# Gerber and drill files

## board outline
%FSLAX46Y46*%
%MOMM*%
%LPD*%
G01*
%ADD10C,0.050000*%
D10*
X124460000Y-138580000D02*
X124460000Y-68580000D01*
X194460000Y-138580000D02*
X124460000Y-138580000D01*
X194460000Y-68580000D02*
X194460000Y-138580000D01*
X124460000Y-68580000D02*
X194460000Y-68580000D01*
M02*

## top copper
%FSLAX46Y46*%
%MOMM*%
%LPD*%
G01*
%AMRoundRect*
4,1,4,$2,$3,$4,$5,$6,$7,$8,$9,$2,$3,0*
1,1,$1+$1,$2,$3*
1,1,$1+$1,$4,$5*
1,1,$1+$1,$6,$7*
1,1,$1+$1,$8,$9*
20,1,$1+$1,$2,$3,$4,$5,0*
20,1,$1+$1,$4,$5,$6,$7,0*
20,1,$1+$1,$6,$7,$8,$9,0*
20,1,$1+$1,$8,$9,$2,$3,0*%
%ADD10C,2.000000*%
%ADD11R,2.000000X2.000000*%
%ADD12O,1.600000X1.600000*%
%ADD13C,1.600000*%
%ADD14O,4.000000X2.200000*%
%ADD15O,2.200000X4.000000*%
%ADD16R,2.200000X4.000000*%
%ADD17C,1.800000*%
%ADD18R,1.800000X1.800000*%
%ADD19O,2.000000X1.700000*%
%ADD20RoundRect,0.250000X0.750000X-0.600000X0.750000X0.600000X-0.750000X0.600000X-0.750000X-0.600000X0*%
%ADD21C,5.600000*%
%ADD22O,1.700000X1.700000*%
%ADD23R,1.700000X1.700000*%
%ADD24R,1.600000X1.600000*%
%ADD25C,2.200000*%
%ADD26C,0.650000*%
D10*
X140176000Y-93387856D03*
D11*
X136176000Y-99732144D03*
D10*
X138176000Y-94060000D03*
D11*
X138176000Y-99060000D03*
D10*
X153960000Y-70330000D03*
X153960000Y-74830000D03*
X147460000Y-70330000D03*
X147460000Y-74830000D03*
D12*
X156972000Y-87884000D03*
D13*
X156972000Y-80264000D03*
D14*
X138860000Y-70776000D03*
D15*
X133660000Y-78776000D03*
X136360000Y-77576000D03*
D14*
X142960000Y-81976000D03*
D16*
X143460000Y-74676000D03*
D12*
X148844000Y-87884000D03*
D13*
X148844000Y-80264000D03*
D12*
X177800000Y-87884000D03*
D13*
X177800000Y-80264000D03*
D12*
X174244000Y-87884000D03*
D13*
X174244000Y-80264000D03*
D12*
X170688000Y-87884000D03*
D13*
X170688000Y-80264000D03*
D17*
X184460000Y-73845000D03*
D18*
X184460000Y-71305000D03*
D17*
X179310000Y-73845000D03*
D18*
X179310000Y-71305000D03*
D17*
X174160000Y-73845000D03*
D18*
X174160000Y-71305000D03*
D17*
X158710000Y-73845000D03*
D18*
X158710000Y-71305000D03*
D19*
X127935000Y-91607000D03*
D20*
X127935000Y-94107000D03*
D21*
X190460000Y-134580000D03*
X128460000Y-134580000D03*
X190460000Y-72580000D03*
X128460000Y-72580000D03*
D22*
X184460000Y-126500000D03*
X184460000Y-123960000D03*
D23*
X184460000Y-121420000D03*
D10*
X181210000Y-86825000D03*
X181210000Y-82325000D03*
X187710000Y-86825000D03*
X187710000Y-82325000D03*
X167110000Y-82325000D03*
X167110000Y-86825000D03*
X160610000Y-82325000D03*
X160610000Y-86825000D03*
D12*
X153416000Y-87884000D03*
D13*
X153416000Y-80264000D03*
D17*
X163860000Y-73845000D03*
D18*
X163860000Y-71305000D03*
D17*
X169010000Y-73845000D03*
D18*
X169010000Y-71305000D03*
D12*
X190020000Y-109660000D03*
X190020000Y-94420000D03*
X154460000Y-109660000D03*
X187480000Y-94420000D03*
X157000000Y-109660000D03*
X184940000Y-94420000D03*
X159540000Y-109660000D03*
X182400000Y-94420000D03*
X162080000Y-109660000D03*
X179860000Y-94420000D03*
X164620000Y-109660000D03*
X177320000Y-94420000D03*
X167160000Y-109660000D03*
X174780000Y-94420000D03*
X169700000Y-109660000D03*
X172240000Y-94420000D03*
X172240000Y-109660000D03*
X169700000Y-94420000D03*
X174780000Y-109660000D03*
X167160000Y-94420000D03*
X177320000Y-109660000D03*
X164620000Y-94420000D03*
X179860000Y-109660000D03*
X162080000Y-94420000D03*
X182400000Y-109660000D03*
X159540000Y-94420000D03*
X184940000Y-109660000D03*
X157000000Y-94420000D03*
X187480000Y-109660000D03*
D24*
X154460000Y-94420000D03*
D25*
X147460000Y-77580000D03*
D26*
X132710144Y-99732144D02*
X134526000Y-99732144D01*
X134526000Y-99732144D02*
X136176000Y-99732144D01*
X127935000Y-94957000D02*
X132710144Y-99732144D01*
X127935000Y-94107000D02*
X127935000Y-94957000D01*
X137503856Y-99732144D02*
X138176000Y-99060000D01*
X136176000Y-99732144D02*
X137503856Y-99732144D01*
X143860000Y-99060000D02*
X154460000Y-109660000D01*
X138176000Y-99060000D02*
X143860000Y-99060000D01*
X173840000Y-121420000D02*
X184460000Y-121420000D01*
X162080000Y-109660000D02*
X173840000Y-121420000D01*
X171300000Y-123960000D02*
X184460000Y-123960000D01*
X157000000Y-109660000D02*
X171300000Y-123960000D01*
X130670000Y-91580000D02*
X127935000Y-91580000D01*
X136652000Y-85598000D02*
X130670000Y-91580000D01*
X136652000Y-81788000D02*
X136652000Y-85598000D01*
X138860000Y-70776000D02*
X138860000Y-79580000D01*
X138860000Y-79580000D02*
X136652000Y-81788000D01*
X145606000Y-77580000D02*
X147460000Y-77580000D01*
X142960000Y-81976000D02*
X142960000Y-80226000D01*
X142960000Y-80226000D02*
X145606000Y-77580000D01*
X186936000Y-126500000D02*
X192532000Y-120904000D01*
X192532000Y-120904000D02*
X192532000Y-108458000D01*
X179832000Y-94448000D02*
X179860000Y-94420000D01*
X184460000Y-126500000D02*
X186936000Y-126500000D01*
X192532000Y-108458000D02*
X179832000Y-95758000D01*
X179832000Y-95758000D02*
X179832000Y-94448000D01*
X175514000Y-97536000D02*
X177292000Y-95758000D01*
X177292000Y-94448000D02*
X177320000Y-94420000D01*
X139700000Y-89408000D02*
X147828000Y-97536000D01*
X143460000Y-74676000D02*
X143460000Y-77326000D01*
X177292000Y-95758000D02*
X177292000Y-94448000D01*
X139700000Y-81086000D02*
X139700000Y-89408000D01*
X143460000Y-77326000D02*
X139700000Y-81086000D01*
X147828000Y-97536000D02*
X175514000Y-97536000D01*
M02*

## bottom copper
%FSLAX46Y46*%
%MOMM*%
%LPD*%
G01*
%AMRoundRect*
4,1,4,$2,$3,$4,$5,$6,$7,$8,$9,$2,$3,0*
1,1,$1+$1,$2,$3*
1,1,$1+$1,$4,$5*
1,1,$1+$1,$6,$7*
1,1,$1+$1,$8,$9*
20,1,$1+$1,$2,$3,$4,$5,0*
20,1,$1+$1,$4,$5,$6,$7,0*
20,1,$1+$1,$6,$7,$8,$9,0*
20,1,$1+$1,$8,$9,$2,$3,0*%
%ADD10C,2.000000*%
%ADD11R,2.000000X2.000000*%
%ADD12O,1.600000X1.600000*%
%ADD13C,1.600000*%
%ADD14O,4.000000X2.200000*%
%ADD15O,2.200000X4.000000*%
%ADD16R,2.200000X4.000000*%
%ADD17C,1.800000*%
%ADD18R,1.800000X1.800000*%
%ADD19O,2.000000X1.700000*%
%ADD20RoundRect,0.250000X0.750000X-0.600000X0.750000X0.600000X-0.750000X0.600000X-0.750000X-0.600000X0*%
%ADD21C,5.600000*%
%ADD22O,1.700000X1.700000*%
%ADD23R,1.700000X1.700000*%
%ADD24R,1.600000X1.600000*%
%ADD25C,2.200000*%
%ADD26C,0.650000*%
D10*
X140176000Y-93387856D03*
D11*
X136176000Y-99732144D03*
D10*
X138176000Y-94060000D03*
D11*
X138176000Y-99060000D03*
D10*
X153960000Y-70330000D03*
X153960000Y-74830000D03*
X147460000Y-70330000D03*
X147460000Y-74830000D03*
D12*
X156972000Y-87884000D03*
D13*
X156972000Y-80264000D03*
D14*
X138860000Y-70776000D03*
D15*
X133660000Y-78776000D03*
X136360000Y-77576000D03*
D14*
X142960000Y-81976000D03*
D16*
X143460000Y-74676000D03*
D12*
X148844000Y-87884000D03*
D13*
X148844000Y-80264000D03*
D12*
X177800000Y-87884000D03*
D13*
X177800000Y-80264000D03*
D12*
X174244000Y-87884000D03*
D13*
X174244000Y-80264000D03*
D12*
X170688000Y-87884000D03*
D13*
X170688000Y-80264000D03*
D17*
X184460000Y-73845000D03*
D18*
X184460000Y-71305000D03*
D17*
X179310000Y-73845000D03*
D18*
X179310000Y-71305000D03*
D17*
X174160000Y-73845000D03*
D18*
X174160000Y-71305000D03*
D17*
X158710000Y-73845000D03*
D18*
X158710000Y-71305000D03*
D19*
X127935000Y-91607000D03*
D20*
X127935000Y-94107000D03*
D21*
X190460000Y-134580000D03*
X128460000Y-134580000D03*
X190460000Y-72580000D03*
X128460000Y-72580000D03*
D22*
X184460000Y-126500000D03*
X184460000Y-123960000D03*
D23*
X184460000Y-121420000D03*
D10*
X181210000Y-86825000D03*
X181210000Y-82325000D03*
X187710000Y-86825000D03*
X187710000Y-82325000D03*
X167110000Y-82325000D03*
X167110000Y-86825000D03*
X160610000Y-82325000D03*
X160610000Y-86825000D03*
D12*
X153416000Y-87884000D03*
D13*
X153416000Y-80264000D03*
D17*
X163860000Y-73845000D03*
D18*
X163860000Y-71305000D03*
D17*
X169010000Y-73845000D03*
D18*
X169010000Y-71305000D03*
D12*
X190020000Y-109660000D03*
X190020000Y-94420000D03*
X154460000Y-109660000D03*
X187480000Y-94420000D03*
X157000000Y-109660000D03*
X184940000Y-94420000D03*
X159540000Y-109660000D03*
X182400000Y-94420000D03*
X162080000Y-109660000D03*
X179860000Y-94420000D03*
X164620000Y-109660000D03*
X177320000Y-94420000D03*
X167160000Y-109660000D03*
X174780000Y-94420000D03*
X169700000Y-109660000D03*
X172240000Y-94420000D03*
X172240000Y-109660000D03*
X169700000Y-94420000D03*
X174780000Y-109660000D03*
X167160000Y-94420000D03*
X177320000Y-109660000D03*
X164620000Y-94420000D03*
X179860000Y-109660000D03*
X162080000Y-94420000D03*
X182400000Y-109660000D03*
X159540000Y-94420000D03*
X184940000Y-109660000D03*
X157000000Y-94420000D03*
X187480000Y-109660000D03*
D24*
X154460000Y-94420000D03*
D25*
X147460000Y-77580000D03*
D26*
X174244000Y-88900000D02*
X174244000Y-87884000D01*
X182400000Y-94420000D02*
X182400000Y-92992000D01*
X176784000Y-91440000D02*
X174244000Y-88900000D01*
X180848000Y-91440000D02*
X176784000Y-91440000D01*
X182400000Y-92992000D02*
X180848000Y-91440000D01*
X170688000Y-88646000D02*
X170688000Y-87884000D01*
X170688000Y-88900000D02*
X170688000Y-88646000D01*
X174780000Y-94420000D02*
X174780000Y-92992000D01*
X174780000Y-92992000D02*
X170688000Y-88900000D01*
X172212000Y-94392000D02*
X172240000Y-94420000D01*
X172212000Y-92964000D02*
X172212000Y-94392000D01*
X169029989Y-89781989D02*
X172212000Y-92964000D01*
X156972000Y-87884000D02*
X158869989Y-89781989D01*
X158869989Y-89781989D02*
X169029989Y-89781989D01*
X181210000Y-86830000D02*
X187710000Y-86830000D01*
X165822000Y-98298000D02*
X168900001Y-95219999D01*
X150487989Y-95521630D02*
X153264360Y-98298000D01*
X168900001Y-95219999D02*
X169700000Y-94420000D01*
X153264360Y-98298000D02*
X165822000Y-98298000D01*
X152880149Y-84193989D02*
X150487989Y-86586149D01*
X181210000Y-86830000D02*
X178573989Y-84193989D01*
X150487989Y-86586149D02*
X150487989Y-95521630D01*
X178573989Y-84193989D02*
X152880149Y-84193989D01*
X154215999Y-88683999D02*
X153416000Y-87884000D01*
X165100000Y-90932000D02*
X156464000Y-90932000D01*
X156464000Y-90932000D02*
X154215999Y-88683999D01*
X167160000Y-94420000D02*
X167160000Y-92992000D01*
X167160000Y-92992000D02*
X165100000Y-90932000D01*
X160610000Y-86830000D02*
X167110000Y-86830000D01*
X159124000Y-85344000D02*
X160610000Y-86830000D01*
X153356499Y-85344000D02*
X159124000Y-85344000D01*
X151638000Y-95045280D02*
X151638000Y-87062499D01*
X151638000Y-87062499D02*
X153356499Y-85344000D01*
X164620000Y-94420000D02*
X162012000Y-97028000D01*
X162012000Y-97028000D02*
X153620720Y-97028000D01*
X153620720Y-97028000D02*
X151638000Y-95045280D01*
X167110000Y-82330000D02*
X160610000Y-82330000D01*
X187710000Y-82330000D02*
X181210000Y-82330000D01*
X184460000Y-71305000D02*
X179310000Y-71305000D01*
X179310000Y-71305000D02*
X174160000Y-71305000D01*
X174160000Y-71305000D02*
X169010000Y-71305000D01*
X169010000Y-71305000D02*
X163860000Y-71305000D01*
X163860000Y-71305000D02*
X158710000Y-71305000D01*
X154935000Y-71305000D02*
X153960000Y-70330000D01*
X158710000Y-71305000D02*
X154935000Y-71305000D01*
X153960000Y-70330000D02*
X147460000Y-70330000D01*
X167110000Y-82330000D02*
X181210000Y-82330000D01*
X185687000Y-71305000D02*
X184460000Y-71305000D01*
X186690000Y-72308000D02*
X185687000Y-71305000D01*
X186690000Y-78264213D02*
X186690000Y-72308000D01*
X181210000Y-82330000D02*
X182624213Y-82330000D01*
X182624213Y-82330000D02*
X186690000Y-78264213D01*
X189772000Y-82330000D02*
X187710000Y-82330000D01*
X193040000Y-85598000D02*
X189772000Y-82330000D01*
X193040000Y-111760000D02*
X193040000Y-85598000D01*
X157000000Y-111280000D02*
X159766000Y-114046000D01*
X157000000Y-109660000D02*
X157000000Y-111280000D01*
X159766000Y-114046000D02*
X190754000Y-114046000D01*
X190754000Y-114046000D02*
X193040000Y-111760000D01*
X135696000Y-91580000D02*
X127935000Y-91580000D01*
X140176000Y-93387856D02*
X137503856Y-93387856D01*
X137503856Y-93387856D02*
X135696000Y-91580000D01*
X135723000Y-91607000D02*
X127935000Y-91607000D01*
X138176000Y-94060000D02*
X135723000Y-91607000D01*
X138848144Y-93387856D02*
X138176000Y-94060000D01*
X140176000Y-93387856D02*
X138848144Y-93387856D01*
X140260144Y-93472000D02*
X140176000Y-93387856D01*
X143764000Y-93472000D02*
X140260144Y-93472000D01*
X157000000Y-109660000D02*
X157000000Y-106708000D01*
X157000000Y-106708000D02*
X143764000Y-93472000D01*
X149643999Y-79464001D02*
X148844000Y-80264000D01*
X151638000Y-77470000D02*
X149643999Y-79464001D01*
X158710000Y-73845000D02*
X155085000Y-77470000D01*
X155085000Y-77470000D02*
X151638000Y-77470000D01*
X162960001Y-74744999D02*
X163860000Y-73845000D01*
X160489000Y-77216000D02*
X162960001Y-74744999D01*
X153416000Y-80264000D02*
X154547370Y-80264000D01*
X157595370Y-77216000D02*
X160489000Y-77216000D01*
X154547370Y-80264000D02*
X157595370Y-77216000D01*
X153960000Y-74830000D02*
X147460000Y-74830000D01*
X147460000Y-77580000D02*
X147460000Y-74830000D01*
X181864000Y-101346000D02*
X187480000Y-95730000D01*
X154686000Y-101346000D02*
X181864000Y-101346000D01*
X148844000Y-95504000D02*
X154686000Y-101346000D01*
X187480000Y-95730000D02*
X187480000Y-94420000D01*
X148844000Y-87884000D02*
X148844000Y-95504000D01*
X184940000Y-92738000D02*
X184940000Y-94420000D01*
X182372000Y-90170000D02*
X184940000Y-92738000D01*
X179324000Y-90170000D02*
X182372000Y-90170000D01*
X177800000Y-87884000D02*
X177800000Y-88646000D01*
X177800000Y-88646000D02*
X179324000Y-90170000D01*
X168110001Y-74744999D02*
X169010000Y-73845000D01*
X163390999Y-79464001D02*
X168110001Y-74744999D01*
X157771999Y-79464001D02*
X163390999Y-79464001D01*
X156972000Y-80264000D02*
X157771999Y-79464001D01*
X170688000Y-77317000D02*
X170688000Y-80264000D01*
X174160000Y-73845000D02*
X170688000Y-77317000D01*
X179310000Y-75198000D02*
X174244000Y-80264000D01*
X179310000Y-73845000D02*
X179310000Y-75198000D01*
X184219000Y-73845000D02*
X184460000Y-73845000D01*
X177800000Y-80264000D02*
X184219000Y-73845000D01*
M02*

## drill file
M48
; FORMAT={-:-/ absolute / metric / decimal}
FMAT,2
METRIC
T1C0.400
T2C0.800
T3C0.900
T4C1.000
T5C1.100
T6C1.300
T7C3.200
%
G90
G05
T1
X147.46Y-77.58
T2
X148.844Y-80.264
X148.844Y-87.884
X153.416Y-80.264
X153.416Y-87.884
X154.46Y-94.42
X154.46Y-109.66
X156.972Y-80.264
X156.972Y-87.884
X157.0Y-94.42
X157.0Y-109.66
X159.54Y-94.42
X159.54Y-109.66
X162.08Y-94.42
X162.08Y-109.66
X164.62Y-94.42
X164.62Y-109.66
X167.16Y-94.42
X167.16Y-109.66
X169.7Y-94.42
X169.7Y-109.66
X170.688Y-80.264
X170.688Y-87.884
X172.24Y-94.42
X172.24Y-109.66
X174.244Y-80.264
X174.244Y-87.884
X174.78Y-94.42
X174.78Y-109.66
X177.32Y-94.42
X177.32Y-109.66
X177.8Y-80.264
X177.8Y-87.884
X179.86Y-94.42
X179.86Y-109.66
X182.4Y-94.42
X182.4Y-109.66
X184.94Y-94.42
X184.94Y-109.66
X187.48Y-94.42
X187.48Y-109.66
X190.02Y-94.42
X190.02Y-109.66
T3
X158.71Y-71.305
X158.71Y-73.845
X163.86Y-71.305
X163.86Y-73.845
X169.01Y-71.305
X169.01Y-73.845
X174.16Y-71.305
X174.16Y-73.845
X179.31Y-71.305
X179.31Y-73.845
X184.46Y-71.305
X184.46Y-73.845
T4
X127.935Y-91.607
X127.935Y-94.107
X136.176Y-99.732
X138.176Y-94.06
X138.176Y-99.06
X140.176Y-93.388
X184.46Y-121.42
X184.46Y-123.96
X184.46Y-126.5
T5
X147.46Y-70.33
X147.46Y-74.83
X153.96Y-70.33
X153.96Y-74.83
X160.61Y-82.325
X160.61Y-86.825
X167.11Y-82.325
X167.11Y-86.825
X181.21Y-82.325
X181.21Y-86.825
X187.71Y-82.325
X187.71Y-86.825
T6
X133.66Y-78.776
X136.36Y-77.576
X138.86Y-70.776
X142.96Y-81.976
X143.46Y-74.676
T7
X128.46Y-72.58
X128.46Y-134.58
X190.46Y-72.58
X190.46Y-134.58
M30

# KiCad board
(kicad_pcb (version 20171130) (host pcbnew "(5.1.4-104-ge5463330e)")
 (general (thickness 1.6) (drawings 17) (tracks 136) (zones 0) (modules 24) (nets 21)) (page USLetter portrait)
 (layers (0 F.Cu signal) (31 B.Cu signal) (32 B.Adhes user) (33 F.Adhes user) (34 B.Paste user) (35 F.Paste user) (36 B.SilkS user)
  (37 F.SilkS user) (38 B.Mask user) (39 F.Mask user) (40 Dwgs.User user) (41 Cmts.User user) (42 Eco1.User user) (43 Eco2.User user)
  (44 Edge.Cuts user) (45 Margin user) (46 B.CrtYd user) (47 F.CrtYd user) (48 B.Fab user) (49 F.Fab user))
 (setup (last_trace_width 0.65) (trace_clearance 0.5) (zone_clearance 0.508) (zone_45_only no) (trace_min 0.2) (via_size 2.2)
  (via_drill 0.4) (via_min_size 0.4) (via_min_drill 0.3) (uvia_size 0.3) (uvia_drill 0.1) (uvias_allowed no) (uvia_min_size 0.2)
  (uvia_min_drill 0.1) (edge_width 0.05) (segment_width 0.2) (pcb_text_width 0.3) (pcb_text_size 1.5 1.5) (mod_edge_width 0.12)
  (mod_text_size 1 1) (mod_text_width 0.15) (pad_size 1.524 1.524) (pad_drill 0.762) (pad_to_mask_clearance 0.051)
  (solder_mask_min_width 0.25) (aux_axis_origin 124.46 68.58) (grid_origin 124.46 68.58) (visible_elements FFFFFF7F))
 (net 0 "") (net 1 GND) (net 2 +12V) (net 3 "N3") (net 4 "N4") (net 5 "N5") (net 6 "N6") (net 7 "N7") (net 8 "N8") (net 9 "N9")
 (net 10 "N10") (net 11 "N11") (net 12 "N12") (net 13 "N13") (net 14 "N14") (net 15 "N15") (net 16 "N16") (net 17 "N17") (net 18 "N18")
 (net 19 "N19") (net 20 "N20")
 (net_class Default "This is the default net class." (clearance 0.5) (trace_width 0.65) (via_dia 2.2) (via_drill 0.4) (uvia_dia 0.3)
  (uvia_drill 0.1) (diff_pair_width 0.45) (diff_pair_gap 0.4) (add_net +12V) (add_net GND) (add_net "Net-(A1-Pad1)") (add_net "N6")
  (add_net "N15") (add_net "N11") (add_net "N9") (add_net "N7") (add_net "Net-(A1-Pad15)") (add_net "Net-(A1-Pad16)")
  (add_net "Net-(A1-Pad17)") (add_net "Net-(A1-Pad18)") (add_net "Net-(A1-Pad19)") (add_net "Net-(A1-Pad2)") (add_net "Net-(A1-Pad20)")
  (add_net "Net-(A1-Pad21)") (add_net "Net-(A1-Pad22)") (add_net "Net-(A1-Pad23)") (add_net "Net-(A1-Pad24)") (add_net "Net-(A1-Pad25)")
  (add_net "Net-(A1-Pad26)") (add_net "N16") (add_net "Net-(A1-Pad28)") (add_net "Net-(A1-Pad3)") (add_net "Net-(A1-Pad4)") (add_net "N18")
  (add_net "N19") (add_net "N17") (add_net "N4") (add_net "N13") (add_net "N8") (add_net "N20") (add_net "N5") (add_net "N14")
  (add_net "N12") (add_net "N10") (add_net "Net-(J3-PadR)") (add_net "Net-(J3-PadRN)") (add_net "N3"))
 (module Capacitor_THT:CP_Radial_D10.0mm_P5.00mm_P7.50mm (layer F.Cu) (at 138.176 99.06 90)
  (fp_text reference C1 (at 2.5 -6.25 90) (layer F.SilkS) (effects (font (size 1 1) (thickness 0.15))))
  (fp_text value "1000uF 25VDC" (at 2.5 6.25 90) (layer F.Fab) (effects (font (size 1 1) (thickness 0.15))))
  (pad 2 thru_hole circle (at 5.672144 2 90) (size 2 2) (drill 1) (layers *.Cu *.Mask) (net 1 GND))
  (pad 1 thru_hole rect (at -0.672144 -2 90) (size 2 2) (drill 1) (layers *.Cu *.Mask) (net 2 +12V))
  (pad 2 thru_hole circle (at 5 0 90) (size 2 2) (drill 1) (layers *.Cu *.Mask) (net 1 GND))
  (pad 1 thru_hole rect (at 0 0 90) (size 2 2) (drill 1) (layers *.Cu *.Mask) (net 2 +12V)))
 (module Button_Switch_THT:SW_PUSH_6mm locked (layer F.Cu) (at 147.46 70.33)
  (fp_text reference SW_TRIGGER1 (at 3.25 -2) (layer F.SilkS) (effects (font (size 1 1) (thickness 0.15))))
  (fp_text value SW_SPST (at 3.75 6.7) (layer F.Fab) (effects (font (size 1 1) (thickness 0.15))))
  (pad 1 thru_hole circle (at 6.5 0 90) (size 2 2) (drill 1.1) (layers *.Cu *.Mask) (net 1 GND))
  (pad 2 thru_hole circle (at 6.5 4.5 90) (size 2 2) (drill 1.1) (layers *.Cu *.Mask) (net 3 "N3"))
  (pad 1 thru_hole circle (at 0 0 90) (size 2 2) (drill 1.1) (layers *.Cu *.Mask) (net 1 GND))
  (pad 2 thru_hole circle (at 0 4.5 90) (size 2 2) (drill 1.1) (layers *.Cu *.Mask) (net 3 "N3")))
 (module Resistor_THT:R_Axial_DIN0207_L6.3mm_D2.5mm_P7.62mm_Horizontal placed (layer F.Cu) (at 156.972 80.264 270)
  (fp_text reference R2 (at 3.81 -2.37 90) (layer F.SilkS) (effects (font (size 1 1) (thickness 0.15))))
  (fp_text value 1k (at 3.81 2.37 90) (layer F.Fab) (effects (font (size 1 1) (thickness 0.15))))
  (pad 2 thru_hole oval (at 7.62 0 270) (size 1.6 1.6) (drill 0.8) (layers *.Cu *.Mask) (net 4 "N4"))
  (pad 1 thru_hole circle (at 0 0 270) (size 1.6 1.6) (drill 0.8) (layers *.Cu *.Mask) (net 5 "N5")))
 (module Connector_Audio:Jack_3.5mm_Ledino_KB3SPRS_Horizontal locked (layer B.Cu) (at 143.46 74.676 270)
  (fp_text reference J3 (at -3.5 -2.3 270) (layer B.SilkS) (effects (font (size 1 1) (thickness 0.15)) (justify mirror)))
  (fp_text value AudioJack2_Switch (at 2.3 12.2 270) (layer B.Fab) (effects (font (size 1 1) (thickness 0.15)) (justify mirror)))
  (pad S thru_hole oval (at -3.9 4.6 270) (size 2.2 4) (drill 1.3) (layers *.Cu *.Mask) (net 1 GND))
  (pad R thru_hole oval (at 4.1 9.8 270) (size 4 2.2) (drill 1.3) (layers *.Cu *.Mask))
  (pad RN thru_hole oval (at 2.9 7.1 270) (size 4 2.2) (drill 1.3) (layers *.Cu *.Mask))
  (pad TN thru_hole oval (at 7.3 0.5 180) (size 4 2.2) (drill 1.3) (layers *.Cu *.Mask) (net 3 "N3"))
  (pad T thru_hole rect (at 0 0 270) (size 4 2.2) (drill 1.3) (layers *.Cu *.Mask) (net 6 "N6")))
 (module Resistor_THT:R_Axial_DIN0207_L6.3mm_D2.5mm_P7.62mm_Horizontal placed (layer F.Cu) (at 148.844 80.264 270)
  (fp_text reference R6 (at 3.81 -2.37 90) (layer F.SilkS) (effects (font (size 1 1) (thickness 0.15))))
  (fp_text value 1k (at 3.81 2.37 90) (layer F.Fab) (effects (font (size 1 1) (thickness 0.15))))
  (pad 2 thru_hole oval (at 7.62 0 270) (size 1.6 1.6) (drill 0.8) (layers *.Cu *.Mask) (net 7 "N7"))
  (pad 1 thru_hole circle (at 0 0 270) (size 1.6 1.6) (drill 0.8) (layers *.Cu *.Mask) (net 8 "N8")))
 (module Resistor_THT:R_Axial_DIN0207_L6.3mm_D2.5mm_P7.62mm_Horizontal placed (layer F.Cu) (at 177.8 80.264 270)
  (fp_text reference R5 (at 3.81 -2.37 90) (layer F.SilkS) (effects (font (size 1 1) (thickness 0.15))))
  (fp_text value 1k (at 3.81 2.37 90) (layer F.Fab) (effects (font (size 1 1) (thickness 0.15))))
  (pad 2 thru_hole oval (at 7.62 0 270) (size 1.6 1.6) (drill 0.8) (layers *.Cu *.Mask) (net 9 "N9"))
  (pad 1 thru_hole circle (at 0 0 270) (size 1.6 1.6) (drill 0.8) (layers *.Cu *.Mask) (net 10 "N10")))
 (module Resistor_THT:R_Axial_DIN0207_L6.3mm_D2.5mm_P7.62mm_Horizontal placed (layer F.Cu) (at 174.244 80.264 270)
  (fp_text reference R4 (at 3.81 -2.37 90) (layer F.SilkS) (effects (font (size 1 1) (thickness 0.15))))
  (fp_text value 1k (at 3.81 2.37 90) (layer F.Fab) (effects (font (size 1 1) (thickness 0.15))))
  (pad 2 thru_hole oval (at 7.62 0 270) (size 1.6 1.6) (drill 0.8) (layers *.Cu *.Mask) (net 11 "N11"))
  (pad 1 thru_hole circle (at 0 0 270) (size 1.6 1.6) (drill 0.8) (layers *.Cu *.Mask) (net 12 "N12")))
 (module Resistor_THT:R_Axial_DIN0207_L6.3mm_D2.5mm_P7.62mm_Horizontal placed (layer F.Cu) (at 170.688 80.264 270)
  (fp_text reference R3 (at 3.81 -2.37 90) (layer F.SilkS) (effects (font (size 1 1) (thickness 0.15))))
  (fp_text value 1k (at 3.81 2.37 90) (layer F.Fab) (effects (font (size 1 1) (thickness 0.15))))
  (pad 2 thru_hole oval (at 7.62 0 270) (size 1.6 1.6) (drill 0.8) (layers *.Cu *.Mask) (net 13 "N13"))
  (pad 1 thru_hole circle (at 0 0 270) (size 1.6 1.6) (drill 0.8) (layers *.Cu *.Mask) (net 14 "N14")))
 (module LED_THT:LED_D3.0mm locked (layer F.Cu) (at 184.46 71.305 270)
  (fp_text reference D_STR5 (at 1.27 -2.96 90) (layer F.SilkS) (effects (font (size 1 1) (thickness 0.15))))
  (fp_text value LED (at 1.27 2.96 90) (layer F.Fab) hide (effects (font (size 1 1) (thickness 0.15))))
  (pad 2 thru_hole circle (at 2.54 0 270) (size 1.8 1.8) (drill 0.9) (layers *.Cu *.Mask) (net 10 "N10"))
  (pad 1 thru_hole rect (at 0 0 270) (size 1.8 1.8) (drill 0.9) (layers *.Cu *.Mask) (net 1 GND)))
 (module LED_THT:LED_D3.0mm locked (layer F.Cu) (at 179.31 71.305 270)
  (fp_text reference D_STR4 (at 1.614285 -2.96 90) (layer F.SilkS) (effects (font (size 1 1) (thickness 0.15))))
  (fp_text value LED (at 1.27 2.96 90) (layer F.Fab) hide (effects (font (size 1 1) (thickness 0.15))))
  (pad 2 thru_hole circle (at 2.54 0 270) (size 1.8 1.8) (drill 0.9) (layers *.Cu *.Mask) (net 12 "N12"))
  (pad 1 thru_hole rect (at 0 0 270) (size 1.8 1.8) (drill 0.9) (layers *.Cu *.Mask) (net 1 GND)))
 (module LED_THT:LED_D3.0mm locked (layer F.Cu) (at 174.16 71.305 270)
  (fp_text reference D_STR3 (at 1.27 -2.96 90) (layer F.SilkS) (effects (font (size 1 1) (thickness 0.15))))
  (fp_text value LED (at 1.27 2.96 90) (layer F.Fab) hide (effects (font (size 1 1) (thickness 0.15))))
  (pad 2 thru_hole circle (at 2.54 0 270) (size 1.8 1.8) (drill 0.9) (layers *.Cu *.Mask) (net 14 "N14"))
  (pad 1 thru_hole rect (at 0 0 270) (size 1.8 1.8) (drill 0.9) (layers *.Cu *.Mask) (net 1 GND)))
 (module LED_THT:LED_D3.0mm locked (layer F.Cu) (at 158.71 71.305 270)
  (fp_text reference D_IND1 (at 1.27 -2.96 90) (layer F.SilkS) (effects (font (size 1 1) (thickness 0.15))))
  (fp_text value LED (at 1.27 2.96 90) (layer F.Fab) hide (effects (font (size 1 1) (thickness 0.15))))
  (pad 2 thru_hole circle (at 2.54 0 270) (size 1.8 1.8) (drill 0.9) (layers *.Cu *.Mask) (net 8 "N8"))
  (pad 1 thru_hole rect (at 0 0 270) (size 1.8 1.8) (drill 0.9) (layers *.Cu *.Mask) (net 1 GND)))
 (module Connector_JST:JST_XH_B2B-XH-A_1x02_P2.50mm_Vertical (layer B.Cu) (at 127.935 94.107 90)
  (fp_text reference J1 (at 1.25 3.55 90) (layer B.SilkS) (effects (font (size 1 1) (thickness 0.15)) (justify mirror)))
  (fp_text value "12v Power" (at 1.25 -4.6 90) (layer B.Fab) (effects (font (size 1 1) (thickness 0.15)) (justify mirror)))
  (pad 2 thru_hole oval (at 2.5 0 90) (size 1.7 2) (drill 1) (layers *.Cu *.Mask) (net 1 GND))
  (pad 1 thru_hole roundrect (at 0 0 90) (size 1.7 2) (drill 1) (layers *.Cu *.Mask) (roundrect_rratio 0.147059) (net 2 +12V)))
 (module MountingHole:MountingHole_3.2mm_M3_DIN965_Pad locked (layer F.Cu) (at 190.46 134.58)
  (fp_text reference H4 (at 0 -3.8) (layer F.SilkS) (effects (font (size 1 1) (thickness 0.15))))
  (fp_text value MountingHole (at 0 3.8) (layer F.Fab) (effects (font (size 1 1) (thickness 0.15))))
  (pad 1 thru_hole circle (at 0 0) (size 5.6 5.6) (drill 3.2) (layers *.Cu *.Mask)))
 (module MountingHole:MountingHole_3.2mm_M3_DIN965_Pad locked (layer F.Cu) (at 128.46 134.58)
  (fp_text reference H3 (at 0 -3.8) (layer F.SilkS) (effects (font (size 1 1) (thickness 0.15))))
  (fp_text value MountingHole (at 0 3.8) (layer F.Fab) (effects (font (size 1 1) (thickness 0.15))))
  (pad 1 thru_hole circle (at 0 0) (size 5.6 5.6) (drill 3.2) (layers *.Cu *.Mask)))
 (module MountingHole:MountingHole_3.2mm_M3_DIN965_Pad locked (layer F.Cu) (at 190.46 72.58)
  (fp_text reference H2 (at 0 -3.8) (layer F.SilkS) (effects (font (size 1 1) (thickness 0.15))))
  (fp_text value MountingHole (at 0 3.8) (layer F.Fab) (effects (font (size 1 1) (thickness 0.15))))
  (pad 1 thru_hole circle (at 0 0) (size 5.6 5.6) (drill 3.2) (layers *.Cu *.Mask)))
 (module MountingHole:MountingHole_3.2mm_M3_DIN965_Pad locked (layer F.Cu) (at 128.46 72.58)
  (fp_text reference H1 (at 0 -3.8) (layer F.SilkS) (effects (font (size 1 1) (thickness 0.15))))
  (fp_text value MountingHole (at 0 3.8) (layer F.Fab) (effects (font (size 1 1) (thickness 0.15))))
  (pad 1 thru_hole circle (at 0 0) (size 5.6 5.6) (drill 3.2) (layers *.Cu *.Mask)))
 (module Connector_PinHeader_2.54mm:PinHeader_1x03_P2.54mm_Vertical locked (layer B.Cu) (at 184.46 121.42 180)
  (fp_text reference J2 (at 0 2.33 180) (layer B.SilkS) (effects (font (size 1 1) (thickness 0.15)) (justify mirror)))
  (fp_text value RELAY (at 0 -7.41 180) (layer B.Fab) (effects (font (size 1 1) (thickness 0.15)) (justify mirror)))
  (pad 3 thru_hole oval (at 0 -5.08 180) (size 1.7 1.7) (drill 1) (layers *.Cu *.Mask) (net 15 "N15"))
  (pad 2 thru_hole oval (at 0 -2.54 180) (size 1.7 1.7) (drill 1) (layers *.Cu *.Mask) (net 1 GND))
  (pad 1 thru_hole rect (at 0 0 180) (size 1.7 1.7) (drill 1) (layers *.Cu *.Mask) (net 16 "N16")))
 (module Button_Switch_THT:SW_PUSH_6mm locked (layer F.Cu) (at 187.71 86.825 180)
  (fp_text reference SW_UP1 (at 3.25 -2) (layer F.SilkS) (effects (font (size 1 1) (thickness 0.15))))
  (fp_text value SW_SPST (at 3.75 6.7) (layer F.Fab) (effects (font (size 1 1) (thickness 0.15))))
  (pad 1 thru_hole circle (at 6.5 0 270) (size 2 2) (drill 1.1) (layers *.Cu *.Mask) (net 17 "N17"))
  (pad 2 thru_hole circle (at 6.5 4.5 270) (size 2 2) (drill 1.1) (layers *.Cu *.Mask) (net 1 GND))
  (pad 1 thru_hole circle (at 0 0 270) (size 2 2) (drill 1.1) (layers *.Cu *.Mask) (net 17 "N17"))
  (pad 2 thru_hole circle (at 0 4.5 270) (size 2 2) (drill 1.1) (layers *.Cu *.Mask) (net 1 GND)))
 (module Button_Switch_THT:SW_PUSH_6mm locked (layer F.Cu) (at 167.11 86.825 180)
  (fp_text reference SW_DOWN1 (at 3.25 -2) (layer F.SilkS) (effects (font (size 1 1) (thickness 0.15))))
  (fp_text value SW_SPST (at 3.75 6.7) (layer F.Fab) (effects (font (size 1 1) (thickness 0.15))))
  (pad 2 thru_hole circle (at 0 4.5 270) (size 2 2) (drill 1.1) (layers *.Cu *.Mask) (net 1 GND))
  (pad 1 thru_hole circle (at 0 0 270) (size 2 2) (drill 1.1) (layers *.Cu *.Mask) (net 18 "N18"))
  (pad 2 thru_hole circle (at 6.5 4.5 270) (size 2 2) (drill 1.1) (layers *.Cu *.Mask) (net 1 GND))
  (pad 1 thru_hole circle (at 6.5 0 270) (size 2 2) (drill 1.1) (layers *.Cu *.Mask) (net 18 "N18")))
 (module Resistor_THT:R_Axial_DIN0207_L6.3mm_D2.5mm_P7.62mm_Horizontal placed (layer F.Cu) (at 153.416 80.264 270)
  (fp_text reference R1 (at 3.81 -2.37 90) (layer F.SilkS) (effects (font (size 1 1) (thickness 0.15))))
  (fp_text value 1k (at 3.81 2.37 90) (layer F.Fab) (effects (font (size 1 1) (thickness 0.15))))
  (pad 2 thru_hole oval (at 7.62 0 270) (size 1.6 1.6) (drill 0.8) (layers *.Cu *.Mask) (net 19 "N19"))
  (pad 1 thru_hole circle (at 0 0 270) (size 1.6 1.6) (drill 0.8) (layers *.Cu *.Mask) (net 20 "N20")))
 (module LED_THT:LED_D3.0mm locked (layer F.Cu) (at 163.86 71.305 270)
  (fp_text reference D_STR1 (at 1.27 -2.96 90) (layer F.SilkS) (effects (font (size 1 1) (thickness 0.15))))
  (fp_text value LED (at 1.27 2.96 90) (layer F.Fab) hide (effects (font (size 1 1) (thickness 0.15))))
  (pad 2 thru_hole circle (at 2.54 0 270) (size 1.8 1.8) (drill 0.9) (layers *.Cu *.Mask) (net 20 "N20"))
  (pad 1 thru_hole rect (at 0 0 270) (size 1.8 1.8) (drill 0.9) (layers *.Cu *.Mask) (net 1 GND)))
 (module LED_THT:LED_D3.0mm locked (layer F.Cu) (at 169.01 71.305 270)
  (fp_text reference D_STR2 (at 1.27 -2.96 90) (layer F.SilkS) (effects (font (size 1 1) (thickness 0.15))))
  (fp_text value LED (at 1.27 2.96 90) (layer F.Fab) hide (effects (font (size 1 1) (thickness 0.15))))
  (pad 2 thru_hole circle (at 2.54 0 270) (size 1.8 1.8) (drill 0.9) (layers *.Cu *.Mask) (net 5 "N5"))
  (pad 1 thru_hole rect (at 0 0 270) (size 1.8 1.8) (drill 0.9) (layers *.Cu *.Mask) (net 1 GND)))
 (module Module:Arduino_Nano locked (layer B.Cu) (at 154.46 94.42 270)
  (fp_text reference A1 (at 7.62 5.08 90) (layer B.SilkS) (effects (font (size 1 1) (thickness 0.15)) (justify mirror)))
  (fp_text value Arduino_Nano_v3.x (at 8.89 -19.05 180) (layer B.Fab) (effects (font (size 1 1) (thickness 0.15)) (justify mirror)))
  (pad 16 thru_hole oval (at 15.24 -35.56 270) (size 1.6 1.6) (drill 0.8) (layers *.Cu *.Mask))
  (pad 15 thru_hole oval (at 0 -35.56 270) (size 1.6 1.6) (drill 0.8) (layers *.Cu *.Mask))
  (pad 30 thru_hole oval (at 15.24 0 270) (size 1.6 1.6) (drill 0.8) (layers *.Cu *.Mask) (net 2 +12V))
  (pad 14 thru_hole oval (at 0 -33.02 270) (size 1.6 1.6) (drill 0.8) (layers *.Cu *.Mask) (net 7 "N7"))
  (pad 29 thru_hole oval (at 15.24 -2.54 270) (size 1.6 1.6) (drill 0.8) (layers *.Cu *.Mask) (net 1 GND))
  (pad 13 thru_hole oval (at 0 -30.48 270) (size 1.6 1.6) (drill 0.8) (layers *.Cu *.Mask) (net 9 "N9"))
  (pad 28 thru_hole oval (at 15.24 -5.08 270) (size 1.6 1.6) (drill 0.8) (layers *.Cu *.Mask))
  (pad 12 thru_hole oval (at 0 -27.94 270) (size 1.6 1.6) (drill 0.8) (layers *.Cu *.Mask) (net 11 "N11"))
  (pad 27 thru_hole oval (at 15.24 -7.62 270) (size 1.6 1.6) (drill 0.8) (layers *.Cu *.Mask) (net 16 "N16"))
  (pad 11 thru_hole oval (at 0 -25.4 270) (size 1.6 1.6) (drill 0.8) (layers *.Cu *.Mask) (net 15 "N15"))
  (pad 26 thru_hole oval (at 15.24 -10.16 270) (size 1.6 1.6) (drill 0.8) (layers *.Cu *.Mask))
  (pad 10 thru_hole oval (at 0 -22.86 270) (size 1.6 1.6) (drill 0.8) (layers *.Cu *.Mask) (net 6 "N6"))
  (pad 25 thru_hole oval (at 15.24 -12.7 270) (size 1.6 1.6) (drill 0.8) (layers *.Cu *.Mask))
  (pad 9 thru_hole oval (at 0 -20.32 270) (size 1.6 1.6) (drill 0.8) (layers *.Cu *.Mask) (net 13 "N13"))
  (pad 24 thru_hole oval (at 15.24 -15.24 270) (size 1.6 1.6) (drill 0.8) (layers *.Cu *.Mask))
  (pad 8 thru_hole oval (at 0 -17.78 270) (size 1.6 1.6) (drill 0.8) (layers *.Cu *.Mask) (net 4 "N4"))
  (pad 23 thru_hole oval (at 15.24 -17.78 270) (size 1.6 1.6) (drill 0.8) (layers *.Cu *.Mask))
  (pad 7 thru_hole oval (at 0 -15.24 270) (size 1.6 1.6) (drill 0.8) (layers *.Cu *.Mask) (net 17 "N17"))
  (pad 22 thru_hole oval (at 15.24 -20.32 270) (size 1.6 1.6) (drill 0.8) (layers *.Cu *.Mask))
  (pad 6 thru_hole oval (at 0 -12.7 270) (size 1.6 1.6) (drill 0.8) (layers *.Cu *.Mask) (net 19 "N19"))
  (pad 21 thru_hole oval (at 15.24 -22.86 270) (size 1.6 1.6) (drill 0.8) (layers *.Cu *.Mask))
  (pad 5 thru_hole oval (at 0 -10.16 270) (size 1.6 1.6) (drill 0.8) (layers *.Cu *.Mask) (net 18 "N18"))
  (pad 20 thru_hole oval (at 15.24 -25.4 270) (size 1.6 1.6) (drill 0.8) (layers *.Cu *.Mask))
  (pad 4 thru_hole oval (at 0 -7.62 270) (size 1.6 1.6) (drill 0.8) (layers *.Cu *.Mask))
  (pad 19 thru_hole oval (at 15.24 -27.94 270) (size 1.6 1.6) (drill 0.8) (layers *.Cu *.Mask))
  (pad 3 thru_hole oval (at 0 -5.08 270) (size 1.6 1.6) (drill 0.8) (layers *.Cu *.Mask))
  (pad 18 thru_hole oval (at 15.24 -30.48 270) (size 1.6 1.6) (drill 0.8) (layers *.Cu *.Mask))
  (pad 2 thru_hole oval (at 0 -2.54 270) (size 1.6 1.6) (drill 0.8) (layers *.Cu *.Mask))
  (pad 17 thru_hole oval (at 15.24 -33.02 270) (size 1.6 1.6) (drill 0.8) (layers *.Cu *.Mask))
  (pad 1 thru_hole rect (at 0 0 270) (size 1.6 1.6) (drill 0.8) (layers *.Cu *.Mask)))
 (gr_line (start 124.46 138.58) (end 124.46 68.58) (layer Edge.Cuts) (width 0.05))
 (gr_line (start 194.46 138.58) (end 124.46 138.58) (layer Edge.Cuts) (width 0.05))
 (gr_line (start 194.46 68.58) (end 194.46 138.58) (layer Edge.Cuts) (width 0.05))
 (gr_line (start 124.46 68.58) (end 194.46 68.58) (layer Edge.Cuts) (width 0.05))
 (segment (start 132.710144 99.732144) (end 134.526 99.732144) (width 0.65) (layer F.Cu) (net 2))
 (segment (start 134.526 99.732144) (end 136.176 99.732144) (width 0.65) (layer F.Cu) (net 2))
 (segment (start 127.935 94.957) (end 132.710144 99.732144) (width 0.65) (layer F.Cu) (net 2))
 (segment (start 127.935 94.107) (end 127.935 94.957) (width 0.65) (layer F.Cu) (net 2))
 (segment (start 137.503856 99.732144) (end 138.176 99.06) (width 0.65) (layer F.Cu) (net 2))
 (segment (start 136.176 99.732144) (end 137.503856 99.732144) (width 0.65) (layer F.Cu) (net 2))
 (segment (start 143.86 99.06) (end 154.46 109.66) (width 0.65) (layer F.Cu) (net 2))
 (segment (start 138.176 99.06) (end 143.86 99.06) (width 0.65) (layer F.Cu) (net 2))
 (segment (start 174.244 88.9) (end 174.244 87.884) (width 0.65) (layer B.Cu) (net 11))
 (segment (start 182.4 94.42) (end 182.4 92.992) (width 0.65) (layer B.Cu) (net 11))
 (segment (start 176.784 91.44) (end 174.244 88.9) (width 0.65) (layer B.Cu) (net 11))
 (segment (start 180.848 91.44) (end 176.784 91.44) (width 0.65) (layer B.Cu) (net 11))
 (segment (start 182.4 92.992) (end 180.848 91.44) (width 0.65) (layer B.Cu) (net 11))
 (segment (start 173.84 121.42) (end 184.46 121.42) (width 0.65) (layer F.Cu) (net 16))
 (segment (start 162.08 109.66) (end 173.84 121.42) (width 0.65) (layer F.Cu) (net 16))
 (segment (start 170.688 88.646) (end 170.688 87.884) (width 0.65) (layer B.Cu) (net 13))
 (segment (start 170.688 88.9) (end 170.688 88.646) (width 0.65) (layer B.Cu) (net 13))
 (segment (start 174.78 94.42) (end 174.78 92.992) (width 0.65) (layer B.Cu) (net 13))
 (segment (start 174.78 92.992) (end 170.688 88.9) (width 0.65) (layer B.Cu) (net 13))
 (segment (start 172.212 94.392) (end 172.24 94.42) (width 0.65) (layer B.Cu) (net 4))
 (segment (start 172.212 92.964) (end 172.212 94.392) (width 0.65) (layer B.Cu) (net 4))
 (segment (start 169.029989 89.781989) (end 172.212 92.964) (width 0.65) (layer B.Cu) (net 4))
 (segment (start 156.972 87.884) (end 158.869989 89.781989) (width 0.65) (layer B.Cu) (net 4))
 (segment (start 158.869989 89.781989) (end 169.029989 89.781989) (width 0.65) (layer B.Cu) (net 4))
 (segment (start 181.21 86.83) (end 187.71 86.83) (width 0.65) (layer B.Cu) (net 17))
 (segment (start 165.822 98.298) (end 168.900001 95.219999) (width 0.65) (layer B.Cu) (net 17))
 (segment (start 150.487989 95.52163) (end 153.26436 98.298) (width 0.65) (layer B.Cu) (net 17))
 (segment (start 168.900001 95.219999) (end 169.7 94.42) (width 0.65) (layer B.Cu) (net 17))
 (segment (start 153.26436 98.298) (end 165.822 98.298) (width 0.65) (layer B.Cu) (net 17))
 (segment (start 152.880149 84.193989) (end 150.487989 86.586149) (width 0.65) (layer B.Cu) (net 17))
 (segment (start 181.21 86.83) (end 178.573989 84.193989) (width 0.65) (layer B.Cu) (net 17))
 (segment (start 150.487989 86.586149) (end 150.487989 95.52163) (width 0.65) (layer B.Cu) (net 17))
 (segment (start 178.573989 84.193989) (end 152.880149 84.193989) (width 0.65) (layer B.Cu) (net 17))
 (segment (start 154.215999 88.683999) (end 153.416 87.884) (width 0.65) (layer B.Cu) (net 19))
 (segment (start 165.1 90.932) (end 156.464 90.932) (width 0.65) (layer B.Cu) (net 19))
 (segment (start 156.464 90.932) (end 154.215999 88.683999) (width 0.65) (layer B.Cu) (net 19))
 (segment (start 167.16 94.42) (end 167.16 92.992) (width 0.65) (layer B.Cu) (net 19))
 (segment (start 167.16 92.992) (end 165.1 90.932) (width 0.65) (layer B.Cu) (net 19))
 (segment (start 160.61 86.83) (end 167.11 86.83) (width 0.65) (layer B.Cu) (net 18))
 (segment (start 159.124 85.344) (end 160.61 86.83) (width 0.65) (layer B.Cu) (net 18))
 (segment (start 153.356499 85.344) (end 159.124 85.344) (width 0.65) (layer B.Cu) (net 18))
 (segment (start 151.638 95.04528) (end 151.638 87.062499) (width 0.65) (layer B.Cu) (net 18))
 (segment (start 151.638 87.062499) (end 153.356499 85.344) (width 0.65) (layer B.Cu) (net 18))
 (segment (start 164.62 94.42) (end 162.012 97.028) (width 0.65) (layer B.Cu) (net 18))
 (segment (start 162.012 97.028) (end 153.62072 97.028) (width 0.65) (layer B.Cu) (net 18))
 (segment (start 153.62072 97.028) (end 151.638 95.04528) (width 0.65) (layer B.Cu) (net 18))
 (segment (start 167.11 82.33) (end 160.61 82.33) (width 0.65) (layer B.Cu) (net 1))
 (segment (start 187.71 82.33) (end 181.21 82.33) (width 0.65) (layer B.Cu) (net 1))
 (segment (start 184.46 71.305) (end 179.31 71.305) (width 0.65) (layer B.Cu) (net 1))
 (segment (start 179.31 71.305) (end 174.16 71.305) (width 0.65) (layer B.Cu) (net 1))
 (segment (start 174.16 71.305) (end 169.01 71.305) (width 0.65) (layer B.Cu) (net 1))
 (segment (start 169.01 71.305) (end 163.86 71.305) (width 0.65) (layer B.Cu) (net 1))
 (segment (start 163.86 71.305) (end 158.71 71.305) (width 0.65) (layer B.Cu) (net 1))
 (segment (start 154.935 71.305) (end 153.96 70.33) (width 0.65) (layer B.Cu) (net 1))
 (segment (start 158.71 71.305) (end 154.935 71.305) (width 0.65) (layer B.Cu) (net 1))
 (segment (start 153.96 70.33) (end 147.46 70.33) (width 0.65) (layer B.Cu) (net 1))
 (segment (start 167.11 82.33) (end 181.21 82.33) (width 0.65) (layer B.Cu) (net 1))
 (segment (start 185.687 71.305) (end 184.46 71.305) (width 0.65) (layer B.Cu) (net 1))
 (segment (start 186.69 72.308) (end 185.687 71.305) (width 0.65) (layer B.Cu) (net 1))
 (segment (start 186.69 78.264213) (end 186.69 72.308) (width 0.65) (layer B.Cu) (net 1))
 (segment (start 181.21 82.33) (end 182.624213 82.33) (width 0.65) (layer B.Cu) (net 1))
 (segment (start 182.624213 82.33) (end 186.69 78.264213) (width 0.65) (layer B.Cu) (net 1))
 (segment (start 171.3 123.96) (end 184.46 123.96) (width 0.65) (layer F.Cu) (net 1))
 (segment (start 157 109.66) (end 171.3 123.96) (width 0.65) (layer F.Cu) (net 1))
 (segment (start 189.772 82.33) (end 187.71 82.33) (width 0.65) (layer B.Cu) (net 1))
 (segment (start 193.04 85.598) (end 189.772 82.33) (width 0.65) (layer B.Cu) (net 1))
 (segment (start 193.04 111.76) (end 193.04 85.598) (width 0.65) (layer B.Cu) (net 1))
 (segment (start 157 111.28) (end 159.766 114.046) (width 0.65) (layer B.Cu) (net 1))
 (segment (start 157 109.66) (end 157 111.28) (width 0.65) (layer B.Cu) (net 1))
 (segment (start 159.766 114.046) (end 190.754 114.046) (width 0.65) (layer B.Cu) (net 1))
 (segment (start 190.754 114.046) (end 193.04 111.76) (width 0.65) (layer B.Cu) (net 1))
 (segment (start 130.67 91.58) (end 127.935 91.58) (width 0.65) (layer F.Cu) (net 1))
 (segment (start 136.652 85.598) (end 130.67 91.58) (width 0.65) (layer F.Cu) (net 1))
 (segment (start 136.652 81.788) (end 136.652 85.598) (width 0.65) (layer F.Cu) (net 1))
 (segment (start 138.86 70.776) (end 138.86 79.58) (width 0.65) (layer F.Cu) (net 1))
 (segment (start 138.86 79.58) (end 136.652 81.788) (width 0.65) (layer F.Cu) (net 1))
 (segment (start 135.696 91.58) (end 127.935 91.58) (width 0.65) (layer B.Cu) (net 1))
 (segment (start 140.176 93.387856) (end 137.503856 93.387856) (width 0.65) (layer B.Cu) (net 1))
 (segment (start 137.503856 93.387856) (end 135.696 91.58) (width 0.65) (layer B.Cu) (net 1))
 (segment (start 135.723 91.607) (end 127.935 91.607) (width 0.65) (layer B.Cu) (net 1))
 (segment (start 138.176 94.06) (end 135.723 91.607) (width 0.65) (layer B.Cu) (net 1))
 (segment (start 138.848144 93.387856) (end 138.176 94.06) (width 0.65) (layer B.Cu) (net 1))
 (segment (start 140.176 93.387856) (end 138.848144 93.387856) (width 0.65) (layer B.Cu) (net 1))
 (segment (start 140.260144 93.472) (end 140.176 93.387856) (width 0.65) (layer B.Cu) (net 1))
 (segment (start 143.764 93.472) (end 140.260144 93.472) (width 0.65) (layer B.Cu) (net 1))
 (segment (start 157 109.66) (end 157 106.708) (width 0.65) (layer B.Cu) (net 1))
 (segment (start 157 106.708) (end 143.764 93.472) (width 0.65) (layer B.Cu) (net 1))
 (segment (start 149.643999 79.464001) (end 148.844 80.264) (width 0.65) (layer B.Cu) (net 8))
 (segment (start 151.638 77.47) (end 149.643999 79.464001) (width 0.65) (layer B.Cu) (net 8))
 (segment (start 158.71 73.845) (end 155.085 77.47) (width 0.65) (layer B.Cu) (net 8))
 (segment (start 155.085 77.47) (end 151.638 77.47) (width 0.65) (layer B.Cu) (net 8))
 (segment (start 162.960001 74.744999) (end 163.86 73.845) (width 0.65) (layer B.Cu) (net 20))
 (segment (start 160.489 77.216) (end 162.960001 74.744999) (width 0.65) (layer B.Cu) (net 20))
 (segment (start 153.416 80.264) (end 154.54737 80.264) (width 0.65) (layer B.Cu) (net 20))
 (segment (start 157.59537 77.216) (end 160.489 77.216) (width 0.65) (layer B.Cu) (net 20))
 (segment (start 154.54737 80.264) (end 157.59537 77.216) (width 0.65) (layer B.Cu) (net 20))
 (segment (start 153.96 74.83) (end 147.46 74.83) (width 0.65) (layer B.Cu) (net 3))
 (segment (start 145.606 77.58) (end 147.46 77.58) (width 0.65) (layer F.Cu) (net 3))
 (segment (start 142.96 81.976) (end 142.96 80.226) (width 0.65) (layer F.Cu) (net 3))
 (via (at 147.46 77.58) (size 2.2) (drill 0.4) (layers F.Cu B.Cu) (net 3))
 (segment (start 142.96 80.226) (end 145.606 77.58) (width 0.65) (layer F.Cu) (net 3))
 (segment (start 147.46 77.58) (end 147.46 74.83) (width 0.65) (layer B.Cu) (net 3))
 (segment (start 181.864 101.346) (end 187.48 95.73) (width 0.65) (layer B.Cu) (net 7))
 (segment (start 154.686 101.346) (end 181.864 101.346) (width 0.65) (layer B.Cu) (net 7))
 (segment (start 148.844 95.504) (end 154.686 101.346) (width 0.65) (layer B.Cu) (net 7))
 (segment (start 187.48 95.73) (end 187.48 94.42) (width 0.65) (layer B.Cu) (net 7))
 (segment (start 148.844 87.884) (end 148.844 95.504) (width 0.65) (layer B.Cu) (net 7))
 (segment (start 184.94 92.738) (end 184.94 94.42) (width 0.65) (layer B.Cu) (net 9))
 (segment (start 182.372 90.17) (end 184.94 92.738) (width 0.65) (layer B.Cu) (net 9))
 (segment (start 179.324 90.17) (end 182.372 90.17) (width 0.65) (layer B.Cu) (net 9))
 (segment (start 177.8 87.884) (end 177.8 88.646) (width 0.65) (layer B.Cu) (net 9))
 (segment (start 177.8 88.646) (end 179.324 90.17) (width 0.65) (layer B.Cu) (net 9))
 (segment (start 186.936 126.5) (end 192.532 120.904) (width 0.65) (layer F.Cu) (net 15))
 (segment (start 192.532 120.904) (end 192.532 108.458) (width 0.65) (layer F.Cu) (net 15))
 (segment (start 179.832 94.448) (end 179.86 94.42) (width 0.65) (layer F.Cu) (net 15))
 (segment (start 184.46 126.5) (end 186.936 126.5) (width 0.65) (layer F.Cu) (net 15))
 (segment (start 192.532 108.458) (end 179.832 95.758) (width 0.65) (layer F.Cu) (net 15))
 (segment (start 179.832 95.758) (end 179.832 94.448) (width 0.65) (layer F.Cu) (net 15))
 (segment (start 175.514 97.536) (end 177.292 95.758) (width 0.65) (layer F.Cu) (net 6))
 (segment (start 177.292 94.448) (end 177.32 94.42) (width 0.65) (layer F.Cu) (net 6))
 (segment (start 139.7 89.408) (end 147.828 97.536) (width 0.65) (layer F.Cu) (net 6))
 (segment (start 143.46 74.676) (end 143.46 77.326) (width 0.65) (layer F.Cu) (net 6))
 (segment (start 177.292 95.758) (end 177.292 94.448) (width 0.65) (layer F.Cu) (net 6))
 (segment (start 139.7 81.086) (end 139.7 89.408) (width 0.65) (layer F.Cu) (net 6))
 (segment (start 143.46 77.326) (end 139.7 81.086) (width 0.65) (layer F.Cu) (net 6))
 (segment (start 147.828 97.536) (end 175.514 97.536) (width 0.65) (layer F.Cu) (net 6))
 (segment (start 168.110001 74.744999) (end 169.01 73.845) (width 0.65) (layer B.Cu) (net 5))
 (segment (start 163.390999 79.464001) (end 168.110001 74.744999) (width 0.65) (layer B.Cu) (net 5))
 (segment (start 157.771999 79.464001) (end 163.390999 79.464001) (width 0.65) (layer B.Cu) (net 5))
 (segment (start 156.972 80.264) (end 157.771999 79.464001) (width 0.65) (layer B.Cu) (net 5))
 (segment (start 170.688 77.317) (end 170.688 80.264) (width 0.65) (layer B.Cu) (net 14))
 (segment (start 174.16 73.845) (end 170.688 77.317) (width 0.65) (layer B.Cu) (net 14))
 (segment (start 179.31 75.198) (end 174.244 80.264) (width 0.65) (layer B.Cu) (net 12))
 (segment (start 179.31 73.845) (end 179.31 75.198) (width 0.65) (layer B.Cu) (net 12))
 (segment (start 184.219 73.845) (end 184.46 73.845) (width 0.65) (layer B.Cu) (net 10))
 (segment (start 177.8 80.264) (end 184.219 73.845) (width 0.65) (layer B.Cu) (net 10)))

